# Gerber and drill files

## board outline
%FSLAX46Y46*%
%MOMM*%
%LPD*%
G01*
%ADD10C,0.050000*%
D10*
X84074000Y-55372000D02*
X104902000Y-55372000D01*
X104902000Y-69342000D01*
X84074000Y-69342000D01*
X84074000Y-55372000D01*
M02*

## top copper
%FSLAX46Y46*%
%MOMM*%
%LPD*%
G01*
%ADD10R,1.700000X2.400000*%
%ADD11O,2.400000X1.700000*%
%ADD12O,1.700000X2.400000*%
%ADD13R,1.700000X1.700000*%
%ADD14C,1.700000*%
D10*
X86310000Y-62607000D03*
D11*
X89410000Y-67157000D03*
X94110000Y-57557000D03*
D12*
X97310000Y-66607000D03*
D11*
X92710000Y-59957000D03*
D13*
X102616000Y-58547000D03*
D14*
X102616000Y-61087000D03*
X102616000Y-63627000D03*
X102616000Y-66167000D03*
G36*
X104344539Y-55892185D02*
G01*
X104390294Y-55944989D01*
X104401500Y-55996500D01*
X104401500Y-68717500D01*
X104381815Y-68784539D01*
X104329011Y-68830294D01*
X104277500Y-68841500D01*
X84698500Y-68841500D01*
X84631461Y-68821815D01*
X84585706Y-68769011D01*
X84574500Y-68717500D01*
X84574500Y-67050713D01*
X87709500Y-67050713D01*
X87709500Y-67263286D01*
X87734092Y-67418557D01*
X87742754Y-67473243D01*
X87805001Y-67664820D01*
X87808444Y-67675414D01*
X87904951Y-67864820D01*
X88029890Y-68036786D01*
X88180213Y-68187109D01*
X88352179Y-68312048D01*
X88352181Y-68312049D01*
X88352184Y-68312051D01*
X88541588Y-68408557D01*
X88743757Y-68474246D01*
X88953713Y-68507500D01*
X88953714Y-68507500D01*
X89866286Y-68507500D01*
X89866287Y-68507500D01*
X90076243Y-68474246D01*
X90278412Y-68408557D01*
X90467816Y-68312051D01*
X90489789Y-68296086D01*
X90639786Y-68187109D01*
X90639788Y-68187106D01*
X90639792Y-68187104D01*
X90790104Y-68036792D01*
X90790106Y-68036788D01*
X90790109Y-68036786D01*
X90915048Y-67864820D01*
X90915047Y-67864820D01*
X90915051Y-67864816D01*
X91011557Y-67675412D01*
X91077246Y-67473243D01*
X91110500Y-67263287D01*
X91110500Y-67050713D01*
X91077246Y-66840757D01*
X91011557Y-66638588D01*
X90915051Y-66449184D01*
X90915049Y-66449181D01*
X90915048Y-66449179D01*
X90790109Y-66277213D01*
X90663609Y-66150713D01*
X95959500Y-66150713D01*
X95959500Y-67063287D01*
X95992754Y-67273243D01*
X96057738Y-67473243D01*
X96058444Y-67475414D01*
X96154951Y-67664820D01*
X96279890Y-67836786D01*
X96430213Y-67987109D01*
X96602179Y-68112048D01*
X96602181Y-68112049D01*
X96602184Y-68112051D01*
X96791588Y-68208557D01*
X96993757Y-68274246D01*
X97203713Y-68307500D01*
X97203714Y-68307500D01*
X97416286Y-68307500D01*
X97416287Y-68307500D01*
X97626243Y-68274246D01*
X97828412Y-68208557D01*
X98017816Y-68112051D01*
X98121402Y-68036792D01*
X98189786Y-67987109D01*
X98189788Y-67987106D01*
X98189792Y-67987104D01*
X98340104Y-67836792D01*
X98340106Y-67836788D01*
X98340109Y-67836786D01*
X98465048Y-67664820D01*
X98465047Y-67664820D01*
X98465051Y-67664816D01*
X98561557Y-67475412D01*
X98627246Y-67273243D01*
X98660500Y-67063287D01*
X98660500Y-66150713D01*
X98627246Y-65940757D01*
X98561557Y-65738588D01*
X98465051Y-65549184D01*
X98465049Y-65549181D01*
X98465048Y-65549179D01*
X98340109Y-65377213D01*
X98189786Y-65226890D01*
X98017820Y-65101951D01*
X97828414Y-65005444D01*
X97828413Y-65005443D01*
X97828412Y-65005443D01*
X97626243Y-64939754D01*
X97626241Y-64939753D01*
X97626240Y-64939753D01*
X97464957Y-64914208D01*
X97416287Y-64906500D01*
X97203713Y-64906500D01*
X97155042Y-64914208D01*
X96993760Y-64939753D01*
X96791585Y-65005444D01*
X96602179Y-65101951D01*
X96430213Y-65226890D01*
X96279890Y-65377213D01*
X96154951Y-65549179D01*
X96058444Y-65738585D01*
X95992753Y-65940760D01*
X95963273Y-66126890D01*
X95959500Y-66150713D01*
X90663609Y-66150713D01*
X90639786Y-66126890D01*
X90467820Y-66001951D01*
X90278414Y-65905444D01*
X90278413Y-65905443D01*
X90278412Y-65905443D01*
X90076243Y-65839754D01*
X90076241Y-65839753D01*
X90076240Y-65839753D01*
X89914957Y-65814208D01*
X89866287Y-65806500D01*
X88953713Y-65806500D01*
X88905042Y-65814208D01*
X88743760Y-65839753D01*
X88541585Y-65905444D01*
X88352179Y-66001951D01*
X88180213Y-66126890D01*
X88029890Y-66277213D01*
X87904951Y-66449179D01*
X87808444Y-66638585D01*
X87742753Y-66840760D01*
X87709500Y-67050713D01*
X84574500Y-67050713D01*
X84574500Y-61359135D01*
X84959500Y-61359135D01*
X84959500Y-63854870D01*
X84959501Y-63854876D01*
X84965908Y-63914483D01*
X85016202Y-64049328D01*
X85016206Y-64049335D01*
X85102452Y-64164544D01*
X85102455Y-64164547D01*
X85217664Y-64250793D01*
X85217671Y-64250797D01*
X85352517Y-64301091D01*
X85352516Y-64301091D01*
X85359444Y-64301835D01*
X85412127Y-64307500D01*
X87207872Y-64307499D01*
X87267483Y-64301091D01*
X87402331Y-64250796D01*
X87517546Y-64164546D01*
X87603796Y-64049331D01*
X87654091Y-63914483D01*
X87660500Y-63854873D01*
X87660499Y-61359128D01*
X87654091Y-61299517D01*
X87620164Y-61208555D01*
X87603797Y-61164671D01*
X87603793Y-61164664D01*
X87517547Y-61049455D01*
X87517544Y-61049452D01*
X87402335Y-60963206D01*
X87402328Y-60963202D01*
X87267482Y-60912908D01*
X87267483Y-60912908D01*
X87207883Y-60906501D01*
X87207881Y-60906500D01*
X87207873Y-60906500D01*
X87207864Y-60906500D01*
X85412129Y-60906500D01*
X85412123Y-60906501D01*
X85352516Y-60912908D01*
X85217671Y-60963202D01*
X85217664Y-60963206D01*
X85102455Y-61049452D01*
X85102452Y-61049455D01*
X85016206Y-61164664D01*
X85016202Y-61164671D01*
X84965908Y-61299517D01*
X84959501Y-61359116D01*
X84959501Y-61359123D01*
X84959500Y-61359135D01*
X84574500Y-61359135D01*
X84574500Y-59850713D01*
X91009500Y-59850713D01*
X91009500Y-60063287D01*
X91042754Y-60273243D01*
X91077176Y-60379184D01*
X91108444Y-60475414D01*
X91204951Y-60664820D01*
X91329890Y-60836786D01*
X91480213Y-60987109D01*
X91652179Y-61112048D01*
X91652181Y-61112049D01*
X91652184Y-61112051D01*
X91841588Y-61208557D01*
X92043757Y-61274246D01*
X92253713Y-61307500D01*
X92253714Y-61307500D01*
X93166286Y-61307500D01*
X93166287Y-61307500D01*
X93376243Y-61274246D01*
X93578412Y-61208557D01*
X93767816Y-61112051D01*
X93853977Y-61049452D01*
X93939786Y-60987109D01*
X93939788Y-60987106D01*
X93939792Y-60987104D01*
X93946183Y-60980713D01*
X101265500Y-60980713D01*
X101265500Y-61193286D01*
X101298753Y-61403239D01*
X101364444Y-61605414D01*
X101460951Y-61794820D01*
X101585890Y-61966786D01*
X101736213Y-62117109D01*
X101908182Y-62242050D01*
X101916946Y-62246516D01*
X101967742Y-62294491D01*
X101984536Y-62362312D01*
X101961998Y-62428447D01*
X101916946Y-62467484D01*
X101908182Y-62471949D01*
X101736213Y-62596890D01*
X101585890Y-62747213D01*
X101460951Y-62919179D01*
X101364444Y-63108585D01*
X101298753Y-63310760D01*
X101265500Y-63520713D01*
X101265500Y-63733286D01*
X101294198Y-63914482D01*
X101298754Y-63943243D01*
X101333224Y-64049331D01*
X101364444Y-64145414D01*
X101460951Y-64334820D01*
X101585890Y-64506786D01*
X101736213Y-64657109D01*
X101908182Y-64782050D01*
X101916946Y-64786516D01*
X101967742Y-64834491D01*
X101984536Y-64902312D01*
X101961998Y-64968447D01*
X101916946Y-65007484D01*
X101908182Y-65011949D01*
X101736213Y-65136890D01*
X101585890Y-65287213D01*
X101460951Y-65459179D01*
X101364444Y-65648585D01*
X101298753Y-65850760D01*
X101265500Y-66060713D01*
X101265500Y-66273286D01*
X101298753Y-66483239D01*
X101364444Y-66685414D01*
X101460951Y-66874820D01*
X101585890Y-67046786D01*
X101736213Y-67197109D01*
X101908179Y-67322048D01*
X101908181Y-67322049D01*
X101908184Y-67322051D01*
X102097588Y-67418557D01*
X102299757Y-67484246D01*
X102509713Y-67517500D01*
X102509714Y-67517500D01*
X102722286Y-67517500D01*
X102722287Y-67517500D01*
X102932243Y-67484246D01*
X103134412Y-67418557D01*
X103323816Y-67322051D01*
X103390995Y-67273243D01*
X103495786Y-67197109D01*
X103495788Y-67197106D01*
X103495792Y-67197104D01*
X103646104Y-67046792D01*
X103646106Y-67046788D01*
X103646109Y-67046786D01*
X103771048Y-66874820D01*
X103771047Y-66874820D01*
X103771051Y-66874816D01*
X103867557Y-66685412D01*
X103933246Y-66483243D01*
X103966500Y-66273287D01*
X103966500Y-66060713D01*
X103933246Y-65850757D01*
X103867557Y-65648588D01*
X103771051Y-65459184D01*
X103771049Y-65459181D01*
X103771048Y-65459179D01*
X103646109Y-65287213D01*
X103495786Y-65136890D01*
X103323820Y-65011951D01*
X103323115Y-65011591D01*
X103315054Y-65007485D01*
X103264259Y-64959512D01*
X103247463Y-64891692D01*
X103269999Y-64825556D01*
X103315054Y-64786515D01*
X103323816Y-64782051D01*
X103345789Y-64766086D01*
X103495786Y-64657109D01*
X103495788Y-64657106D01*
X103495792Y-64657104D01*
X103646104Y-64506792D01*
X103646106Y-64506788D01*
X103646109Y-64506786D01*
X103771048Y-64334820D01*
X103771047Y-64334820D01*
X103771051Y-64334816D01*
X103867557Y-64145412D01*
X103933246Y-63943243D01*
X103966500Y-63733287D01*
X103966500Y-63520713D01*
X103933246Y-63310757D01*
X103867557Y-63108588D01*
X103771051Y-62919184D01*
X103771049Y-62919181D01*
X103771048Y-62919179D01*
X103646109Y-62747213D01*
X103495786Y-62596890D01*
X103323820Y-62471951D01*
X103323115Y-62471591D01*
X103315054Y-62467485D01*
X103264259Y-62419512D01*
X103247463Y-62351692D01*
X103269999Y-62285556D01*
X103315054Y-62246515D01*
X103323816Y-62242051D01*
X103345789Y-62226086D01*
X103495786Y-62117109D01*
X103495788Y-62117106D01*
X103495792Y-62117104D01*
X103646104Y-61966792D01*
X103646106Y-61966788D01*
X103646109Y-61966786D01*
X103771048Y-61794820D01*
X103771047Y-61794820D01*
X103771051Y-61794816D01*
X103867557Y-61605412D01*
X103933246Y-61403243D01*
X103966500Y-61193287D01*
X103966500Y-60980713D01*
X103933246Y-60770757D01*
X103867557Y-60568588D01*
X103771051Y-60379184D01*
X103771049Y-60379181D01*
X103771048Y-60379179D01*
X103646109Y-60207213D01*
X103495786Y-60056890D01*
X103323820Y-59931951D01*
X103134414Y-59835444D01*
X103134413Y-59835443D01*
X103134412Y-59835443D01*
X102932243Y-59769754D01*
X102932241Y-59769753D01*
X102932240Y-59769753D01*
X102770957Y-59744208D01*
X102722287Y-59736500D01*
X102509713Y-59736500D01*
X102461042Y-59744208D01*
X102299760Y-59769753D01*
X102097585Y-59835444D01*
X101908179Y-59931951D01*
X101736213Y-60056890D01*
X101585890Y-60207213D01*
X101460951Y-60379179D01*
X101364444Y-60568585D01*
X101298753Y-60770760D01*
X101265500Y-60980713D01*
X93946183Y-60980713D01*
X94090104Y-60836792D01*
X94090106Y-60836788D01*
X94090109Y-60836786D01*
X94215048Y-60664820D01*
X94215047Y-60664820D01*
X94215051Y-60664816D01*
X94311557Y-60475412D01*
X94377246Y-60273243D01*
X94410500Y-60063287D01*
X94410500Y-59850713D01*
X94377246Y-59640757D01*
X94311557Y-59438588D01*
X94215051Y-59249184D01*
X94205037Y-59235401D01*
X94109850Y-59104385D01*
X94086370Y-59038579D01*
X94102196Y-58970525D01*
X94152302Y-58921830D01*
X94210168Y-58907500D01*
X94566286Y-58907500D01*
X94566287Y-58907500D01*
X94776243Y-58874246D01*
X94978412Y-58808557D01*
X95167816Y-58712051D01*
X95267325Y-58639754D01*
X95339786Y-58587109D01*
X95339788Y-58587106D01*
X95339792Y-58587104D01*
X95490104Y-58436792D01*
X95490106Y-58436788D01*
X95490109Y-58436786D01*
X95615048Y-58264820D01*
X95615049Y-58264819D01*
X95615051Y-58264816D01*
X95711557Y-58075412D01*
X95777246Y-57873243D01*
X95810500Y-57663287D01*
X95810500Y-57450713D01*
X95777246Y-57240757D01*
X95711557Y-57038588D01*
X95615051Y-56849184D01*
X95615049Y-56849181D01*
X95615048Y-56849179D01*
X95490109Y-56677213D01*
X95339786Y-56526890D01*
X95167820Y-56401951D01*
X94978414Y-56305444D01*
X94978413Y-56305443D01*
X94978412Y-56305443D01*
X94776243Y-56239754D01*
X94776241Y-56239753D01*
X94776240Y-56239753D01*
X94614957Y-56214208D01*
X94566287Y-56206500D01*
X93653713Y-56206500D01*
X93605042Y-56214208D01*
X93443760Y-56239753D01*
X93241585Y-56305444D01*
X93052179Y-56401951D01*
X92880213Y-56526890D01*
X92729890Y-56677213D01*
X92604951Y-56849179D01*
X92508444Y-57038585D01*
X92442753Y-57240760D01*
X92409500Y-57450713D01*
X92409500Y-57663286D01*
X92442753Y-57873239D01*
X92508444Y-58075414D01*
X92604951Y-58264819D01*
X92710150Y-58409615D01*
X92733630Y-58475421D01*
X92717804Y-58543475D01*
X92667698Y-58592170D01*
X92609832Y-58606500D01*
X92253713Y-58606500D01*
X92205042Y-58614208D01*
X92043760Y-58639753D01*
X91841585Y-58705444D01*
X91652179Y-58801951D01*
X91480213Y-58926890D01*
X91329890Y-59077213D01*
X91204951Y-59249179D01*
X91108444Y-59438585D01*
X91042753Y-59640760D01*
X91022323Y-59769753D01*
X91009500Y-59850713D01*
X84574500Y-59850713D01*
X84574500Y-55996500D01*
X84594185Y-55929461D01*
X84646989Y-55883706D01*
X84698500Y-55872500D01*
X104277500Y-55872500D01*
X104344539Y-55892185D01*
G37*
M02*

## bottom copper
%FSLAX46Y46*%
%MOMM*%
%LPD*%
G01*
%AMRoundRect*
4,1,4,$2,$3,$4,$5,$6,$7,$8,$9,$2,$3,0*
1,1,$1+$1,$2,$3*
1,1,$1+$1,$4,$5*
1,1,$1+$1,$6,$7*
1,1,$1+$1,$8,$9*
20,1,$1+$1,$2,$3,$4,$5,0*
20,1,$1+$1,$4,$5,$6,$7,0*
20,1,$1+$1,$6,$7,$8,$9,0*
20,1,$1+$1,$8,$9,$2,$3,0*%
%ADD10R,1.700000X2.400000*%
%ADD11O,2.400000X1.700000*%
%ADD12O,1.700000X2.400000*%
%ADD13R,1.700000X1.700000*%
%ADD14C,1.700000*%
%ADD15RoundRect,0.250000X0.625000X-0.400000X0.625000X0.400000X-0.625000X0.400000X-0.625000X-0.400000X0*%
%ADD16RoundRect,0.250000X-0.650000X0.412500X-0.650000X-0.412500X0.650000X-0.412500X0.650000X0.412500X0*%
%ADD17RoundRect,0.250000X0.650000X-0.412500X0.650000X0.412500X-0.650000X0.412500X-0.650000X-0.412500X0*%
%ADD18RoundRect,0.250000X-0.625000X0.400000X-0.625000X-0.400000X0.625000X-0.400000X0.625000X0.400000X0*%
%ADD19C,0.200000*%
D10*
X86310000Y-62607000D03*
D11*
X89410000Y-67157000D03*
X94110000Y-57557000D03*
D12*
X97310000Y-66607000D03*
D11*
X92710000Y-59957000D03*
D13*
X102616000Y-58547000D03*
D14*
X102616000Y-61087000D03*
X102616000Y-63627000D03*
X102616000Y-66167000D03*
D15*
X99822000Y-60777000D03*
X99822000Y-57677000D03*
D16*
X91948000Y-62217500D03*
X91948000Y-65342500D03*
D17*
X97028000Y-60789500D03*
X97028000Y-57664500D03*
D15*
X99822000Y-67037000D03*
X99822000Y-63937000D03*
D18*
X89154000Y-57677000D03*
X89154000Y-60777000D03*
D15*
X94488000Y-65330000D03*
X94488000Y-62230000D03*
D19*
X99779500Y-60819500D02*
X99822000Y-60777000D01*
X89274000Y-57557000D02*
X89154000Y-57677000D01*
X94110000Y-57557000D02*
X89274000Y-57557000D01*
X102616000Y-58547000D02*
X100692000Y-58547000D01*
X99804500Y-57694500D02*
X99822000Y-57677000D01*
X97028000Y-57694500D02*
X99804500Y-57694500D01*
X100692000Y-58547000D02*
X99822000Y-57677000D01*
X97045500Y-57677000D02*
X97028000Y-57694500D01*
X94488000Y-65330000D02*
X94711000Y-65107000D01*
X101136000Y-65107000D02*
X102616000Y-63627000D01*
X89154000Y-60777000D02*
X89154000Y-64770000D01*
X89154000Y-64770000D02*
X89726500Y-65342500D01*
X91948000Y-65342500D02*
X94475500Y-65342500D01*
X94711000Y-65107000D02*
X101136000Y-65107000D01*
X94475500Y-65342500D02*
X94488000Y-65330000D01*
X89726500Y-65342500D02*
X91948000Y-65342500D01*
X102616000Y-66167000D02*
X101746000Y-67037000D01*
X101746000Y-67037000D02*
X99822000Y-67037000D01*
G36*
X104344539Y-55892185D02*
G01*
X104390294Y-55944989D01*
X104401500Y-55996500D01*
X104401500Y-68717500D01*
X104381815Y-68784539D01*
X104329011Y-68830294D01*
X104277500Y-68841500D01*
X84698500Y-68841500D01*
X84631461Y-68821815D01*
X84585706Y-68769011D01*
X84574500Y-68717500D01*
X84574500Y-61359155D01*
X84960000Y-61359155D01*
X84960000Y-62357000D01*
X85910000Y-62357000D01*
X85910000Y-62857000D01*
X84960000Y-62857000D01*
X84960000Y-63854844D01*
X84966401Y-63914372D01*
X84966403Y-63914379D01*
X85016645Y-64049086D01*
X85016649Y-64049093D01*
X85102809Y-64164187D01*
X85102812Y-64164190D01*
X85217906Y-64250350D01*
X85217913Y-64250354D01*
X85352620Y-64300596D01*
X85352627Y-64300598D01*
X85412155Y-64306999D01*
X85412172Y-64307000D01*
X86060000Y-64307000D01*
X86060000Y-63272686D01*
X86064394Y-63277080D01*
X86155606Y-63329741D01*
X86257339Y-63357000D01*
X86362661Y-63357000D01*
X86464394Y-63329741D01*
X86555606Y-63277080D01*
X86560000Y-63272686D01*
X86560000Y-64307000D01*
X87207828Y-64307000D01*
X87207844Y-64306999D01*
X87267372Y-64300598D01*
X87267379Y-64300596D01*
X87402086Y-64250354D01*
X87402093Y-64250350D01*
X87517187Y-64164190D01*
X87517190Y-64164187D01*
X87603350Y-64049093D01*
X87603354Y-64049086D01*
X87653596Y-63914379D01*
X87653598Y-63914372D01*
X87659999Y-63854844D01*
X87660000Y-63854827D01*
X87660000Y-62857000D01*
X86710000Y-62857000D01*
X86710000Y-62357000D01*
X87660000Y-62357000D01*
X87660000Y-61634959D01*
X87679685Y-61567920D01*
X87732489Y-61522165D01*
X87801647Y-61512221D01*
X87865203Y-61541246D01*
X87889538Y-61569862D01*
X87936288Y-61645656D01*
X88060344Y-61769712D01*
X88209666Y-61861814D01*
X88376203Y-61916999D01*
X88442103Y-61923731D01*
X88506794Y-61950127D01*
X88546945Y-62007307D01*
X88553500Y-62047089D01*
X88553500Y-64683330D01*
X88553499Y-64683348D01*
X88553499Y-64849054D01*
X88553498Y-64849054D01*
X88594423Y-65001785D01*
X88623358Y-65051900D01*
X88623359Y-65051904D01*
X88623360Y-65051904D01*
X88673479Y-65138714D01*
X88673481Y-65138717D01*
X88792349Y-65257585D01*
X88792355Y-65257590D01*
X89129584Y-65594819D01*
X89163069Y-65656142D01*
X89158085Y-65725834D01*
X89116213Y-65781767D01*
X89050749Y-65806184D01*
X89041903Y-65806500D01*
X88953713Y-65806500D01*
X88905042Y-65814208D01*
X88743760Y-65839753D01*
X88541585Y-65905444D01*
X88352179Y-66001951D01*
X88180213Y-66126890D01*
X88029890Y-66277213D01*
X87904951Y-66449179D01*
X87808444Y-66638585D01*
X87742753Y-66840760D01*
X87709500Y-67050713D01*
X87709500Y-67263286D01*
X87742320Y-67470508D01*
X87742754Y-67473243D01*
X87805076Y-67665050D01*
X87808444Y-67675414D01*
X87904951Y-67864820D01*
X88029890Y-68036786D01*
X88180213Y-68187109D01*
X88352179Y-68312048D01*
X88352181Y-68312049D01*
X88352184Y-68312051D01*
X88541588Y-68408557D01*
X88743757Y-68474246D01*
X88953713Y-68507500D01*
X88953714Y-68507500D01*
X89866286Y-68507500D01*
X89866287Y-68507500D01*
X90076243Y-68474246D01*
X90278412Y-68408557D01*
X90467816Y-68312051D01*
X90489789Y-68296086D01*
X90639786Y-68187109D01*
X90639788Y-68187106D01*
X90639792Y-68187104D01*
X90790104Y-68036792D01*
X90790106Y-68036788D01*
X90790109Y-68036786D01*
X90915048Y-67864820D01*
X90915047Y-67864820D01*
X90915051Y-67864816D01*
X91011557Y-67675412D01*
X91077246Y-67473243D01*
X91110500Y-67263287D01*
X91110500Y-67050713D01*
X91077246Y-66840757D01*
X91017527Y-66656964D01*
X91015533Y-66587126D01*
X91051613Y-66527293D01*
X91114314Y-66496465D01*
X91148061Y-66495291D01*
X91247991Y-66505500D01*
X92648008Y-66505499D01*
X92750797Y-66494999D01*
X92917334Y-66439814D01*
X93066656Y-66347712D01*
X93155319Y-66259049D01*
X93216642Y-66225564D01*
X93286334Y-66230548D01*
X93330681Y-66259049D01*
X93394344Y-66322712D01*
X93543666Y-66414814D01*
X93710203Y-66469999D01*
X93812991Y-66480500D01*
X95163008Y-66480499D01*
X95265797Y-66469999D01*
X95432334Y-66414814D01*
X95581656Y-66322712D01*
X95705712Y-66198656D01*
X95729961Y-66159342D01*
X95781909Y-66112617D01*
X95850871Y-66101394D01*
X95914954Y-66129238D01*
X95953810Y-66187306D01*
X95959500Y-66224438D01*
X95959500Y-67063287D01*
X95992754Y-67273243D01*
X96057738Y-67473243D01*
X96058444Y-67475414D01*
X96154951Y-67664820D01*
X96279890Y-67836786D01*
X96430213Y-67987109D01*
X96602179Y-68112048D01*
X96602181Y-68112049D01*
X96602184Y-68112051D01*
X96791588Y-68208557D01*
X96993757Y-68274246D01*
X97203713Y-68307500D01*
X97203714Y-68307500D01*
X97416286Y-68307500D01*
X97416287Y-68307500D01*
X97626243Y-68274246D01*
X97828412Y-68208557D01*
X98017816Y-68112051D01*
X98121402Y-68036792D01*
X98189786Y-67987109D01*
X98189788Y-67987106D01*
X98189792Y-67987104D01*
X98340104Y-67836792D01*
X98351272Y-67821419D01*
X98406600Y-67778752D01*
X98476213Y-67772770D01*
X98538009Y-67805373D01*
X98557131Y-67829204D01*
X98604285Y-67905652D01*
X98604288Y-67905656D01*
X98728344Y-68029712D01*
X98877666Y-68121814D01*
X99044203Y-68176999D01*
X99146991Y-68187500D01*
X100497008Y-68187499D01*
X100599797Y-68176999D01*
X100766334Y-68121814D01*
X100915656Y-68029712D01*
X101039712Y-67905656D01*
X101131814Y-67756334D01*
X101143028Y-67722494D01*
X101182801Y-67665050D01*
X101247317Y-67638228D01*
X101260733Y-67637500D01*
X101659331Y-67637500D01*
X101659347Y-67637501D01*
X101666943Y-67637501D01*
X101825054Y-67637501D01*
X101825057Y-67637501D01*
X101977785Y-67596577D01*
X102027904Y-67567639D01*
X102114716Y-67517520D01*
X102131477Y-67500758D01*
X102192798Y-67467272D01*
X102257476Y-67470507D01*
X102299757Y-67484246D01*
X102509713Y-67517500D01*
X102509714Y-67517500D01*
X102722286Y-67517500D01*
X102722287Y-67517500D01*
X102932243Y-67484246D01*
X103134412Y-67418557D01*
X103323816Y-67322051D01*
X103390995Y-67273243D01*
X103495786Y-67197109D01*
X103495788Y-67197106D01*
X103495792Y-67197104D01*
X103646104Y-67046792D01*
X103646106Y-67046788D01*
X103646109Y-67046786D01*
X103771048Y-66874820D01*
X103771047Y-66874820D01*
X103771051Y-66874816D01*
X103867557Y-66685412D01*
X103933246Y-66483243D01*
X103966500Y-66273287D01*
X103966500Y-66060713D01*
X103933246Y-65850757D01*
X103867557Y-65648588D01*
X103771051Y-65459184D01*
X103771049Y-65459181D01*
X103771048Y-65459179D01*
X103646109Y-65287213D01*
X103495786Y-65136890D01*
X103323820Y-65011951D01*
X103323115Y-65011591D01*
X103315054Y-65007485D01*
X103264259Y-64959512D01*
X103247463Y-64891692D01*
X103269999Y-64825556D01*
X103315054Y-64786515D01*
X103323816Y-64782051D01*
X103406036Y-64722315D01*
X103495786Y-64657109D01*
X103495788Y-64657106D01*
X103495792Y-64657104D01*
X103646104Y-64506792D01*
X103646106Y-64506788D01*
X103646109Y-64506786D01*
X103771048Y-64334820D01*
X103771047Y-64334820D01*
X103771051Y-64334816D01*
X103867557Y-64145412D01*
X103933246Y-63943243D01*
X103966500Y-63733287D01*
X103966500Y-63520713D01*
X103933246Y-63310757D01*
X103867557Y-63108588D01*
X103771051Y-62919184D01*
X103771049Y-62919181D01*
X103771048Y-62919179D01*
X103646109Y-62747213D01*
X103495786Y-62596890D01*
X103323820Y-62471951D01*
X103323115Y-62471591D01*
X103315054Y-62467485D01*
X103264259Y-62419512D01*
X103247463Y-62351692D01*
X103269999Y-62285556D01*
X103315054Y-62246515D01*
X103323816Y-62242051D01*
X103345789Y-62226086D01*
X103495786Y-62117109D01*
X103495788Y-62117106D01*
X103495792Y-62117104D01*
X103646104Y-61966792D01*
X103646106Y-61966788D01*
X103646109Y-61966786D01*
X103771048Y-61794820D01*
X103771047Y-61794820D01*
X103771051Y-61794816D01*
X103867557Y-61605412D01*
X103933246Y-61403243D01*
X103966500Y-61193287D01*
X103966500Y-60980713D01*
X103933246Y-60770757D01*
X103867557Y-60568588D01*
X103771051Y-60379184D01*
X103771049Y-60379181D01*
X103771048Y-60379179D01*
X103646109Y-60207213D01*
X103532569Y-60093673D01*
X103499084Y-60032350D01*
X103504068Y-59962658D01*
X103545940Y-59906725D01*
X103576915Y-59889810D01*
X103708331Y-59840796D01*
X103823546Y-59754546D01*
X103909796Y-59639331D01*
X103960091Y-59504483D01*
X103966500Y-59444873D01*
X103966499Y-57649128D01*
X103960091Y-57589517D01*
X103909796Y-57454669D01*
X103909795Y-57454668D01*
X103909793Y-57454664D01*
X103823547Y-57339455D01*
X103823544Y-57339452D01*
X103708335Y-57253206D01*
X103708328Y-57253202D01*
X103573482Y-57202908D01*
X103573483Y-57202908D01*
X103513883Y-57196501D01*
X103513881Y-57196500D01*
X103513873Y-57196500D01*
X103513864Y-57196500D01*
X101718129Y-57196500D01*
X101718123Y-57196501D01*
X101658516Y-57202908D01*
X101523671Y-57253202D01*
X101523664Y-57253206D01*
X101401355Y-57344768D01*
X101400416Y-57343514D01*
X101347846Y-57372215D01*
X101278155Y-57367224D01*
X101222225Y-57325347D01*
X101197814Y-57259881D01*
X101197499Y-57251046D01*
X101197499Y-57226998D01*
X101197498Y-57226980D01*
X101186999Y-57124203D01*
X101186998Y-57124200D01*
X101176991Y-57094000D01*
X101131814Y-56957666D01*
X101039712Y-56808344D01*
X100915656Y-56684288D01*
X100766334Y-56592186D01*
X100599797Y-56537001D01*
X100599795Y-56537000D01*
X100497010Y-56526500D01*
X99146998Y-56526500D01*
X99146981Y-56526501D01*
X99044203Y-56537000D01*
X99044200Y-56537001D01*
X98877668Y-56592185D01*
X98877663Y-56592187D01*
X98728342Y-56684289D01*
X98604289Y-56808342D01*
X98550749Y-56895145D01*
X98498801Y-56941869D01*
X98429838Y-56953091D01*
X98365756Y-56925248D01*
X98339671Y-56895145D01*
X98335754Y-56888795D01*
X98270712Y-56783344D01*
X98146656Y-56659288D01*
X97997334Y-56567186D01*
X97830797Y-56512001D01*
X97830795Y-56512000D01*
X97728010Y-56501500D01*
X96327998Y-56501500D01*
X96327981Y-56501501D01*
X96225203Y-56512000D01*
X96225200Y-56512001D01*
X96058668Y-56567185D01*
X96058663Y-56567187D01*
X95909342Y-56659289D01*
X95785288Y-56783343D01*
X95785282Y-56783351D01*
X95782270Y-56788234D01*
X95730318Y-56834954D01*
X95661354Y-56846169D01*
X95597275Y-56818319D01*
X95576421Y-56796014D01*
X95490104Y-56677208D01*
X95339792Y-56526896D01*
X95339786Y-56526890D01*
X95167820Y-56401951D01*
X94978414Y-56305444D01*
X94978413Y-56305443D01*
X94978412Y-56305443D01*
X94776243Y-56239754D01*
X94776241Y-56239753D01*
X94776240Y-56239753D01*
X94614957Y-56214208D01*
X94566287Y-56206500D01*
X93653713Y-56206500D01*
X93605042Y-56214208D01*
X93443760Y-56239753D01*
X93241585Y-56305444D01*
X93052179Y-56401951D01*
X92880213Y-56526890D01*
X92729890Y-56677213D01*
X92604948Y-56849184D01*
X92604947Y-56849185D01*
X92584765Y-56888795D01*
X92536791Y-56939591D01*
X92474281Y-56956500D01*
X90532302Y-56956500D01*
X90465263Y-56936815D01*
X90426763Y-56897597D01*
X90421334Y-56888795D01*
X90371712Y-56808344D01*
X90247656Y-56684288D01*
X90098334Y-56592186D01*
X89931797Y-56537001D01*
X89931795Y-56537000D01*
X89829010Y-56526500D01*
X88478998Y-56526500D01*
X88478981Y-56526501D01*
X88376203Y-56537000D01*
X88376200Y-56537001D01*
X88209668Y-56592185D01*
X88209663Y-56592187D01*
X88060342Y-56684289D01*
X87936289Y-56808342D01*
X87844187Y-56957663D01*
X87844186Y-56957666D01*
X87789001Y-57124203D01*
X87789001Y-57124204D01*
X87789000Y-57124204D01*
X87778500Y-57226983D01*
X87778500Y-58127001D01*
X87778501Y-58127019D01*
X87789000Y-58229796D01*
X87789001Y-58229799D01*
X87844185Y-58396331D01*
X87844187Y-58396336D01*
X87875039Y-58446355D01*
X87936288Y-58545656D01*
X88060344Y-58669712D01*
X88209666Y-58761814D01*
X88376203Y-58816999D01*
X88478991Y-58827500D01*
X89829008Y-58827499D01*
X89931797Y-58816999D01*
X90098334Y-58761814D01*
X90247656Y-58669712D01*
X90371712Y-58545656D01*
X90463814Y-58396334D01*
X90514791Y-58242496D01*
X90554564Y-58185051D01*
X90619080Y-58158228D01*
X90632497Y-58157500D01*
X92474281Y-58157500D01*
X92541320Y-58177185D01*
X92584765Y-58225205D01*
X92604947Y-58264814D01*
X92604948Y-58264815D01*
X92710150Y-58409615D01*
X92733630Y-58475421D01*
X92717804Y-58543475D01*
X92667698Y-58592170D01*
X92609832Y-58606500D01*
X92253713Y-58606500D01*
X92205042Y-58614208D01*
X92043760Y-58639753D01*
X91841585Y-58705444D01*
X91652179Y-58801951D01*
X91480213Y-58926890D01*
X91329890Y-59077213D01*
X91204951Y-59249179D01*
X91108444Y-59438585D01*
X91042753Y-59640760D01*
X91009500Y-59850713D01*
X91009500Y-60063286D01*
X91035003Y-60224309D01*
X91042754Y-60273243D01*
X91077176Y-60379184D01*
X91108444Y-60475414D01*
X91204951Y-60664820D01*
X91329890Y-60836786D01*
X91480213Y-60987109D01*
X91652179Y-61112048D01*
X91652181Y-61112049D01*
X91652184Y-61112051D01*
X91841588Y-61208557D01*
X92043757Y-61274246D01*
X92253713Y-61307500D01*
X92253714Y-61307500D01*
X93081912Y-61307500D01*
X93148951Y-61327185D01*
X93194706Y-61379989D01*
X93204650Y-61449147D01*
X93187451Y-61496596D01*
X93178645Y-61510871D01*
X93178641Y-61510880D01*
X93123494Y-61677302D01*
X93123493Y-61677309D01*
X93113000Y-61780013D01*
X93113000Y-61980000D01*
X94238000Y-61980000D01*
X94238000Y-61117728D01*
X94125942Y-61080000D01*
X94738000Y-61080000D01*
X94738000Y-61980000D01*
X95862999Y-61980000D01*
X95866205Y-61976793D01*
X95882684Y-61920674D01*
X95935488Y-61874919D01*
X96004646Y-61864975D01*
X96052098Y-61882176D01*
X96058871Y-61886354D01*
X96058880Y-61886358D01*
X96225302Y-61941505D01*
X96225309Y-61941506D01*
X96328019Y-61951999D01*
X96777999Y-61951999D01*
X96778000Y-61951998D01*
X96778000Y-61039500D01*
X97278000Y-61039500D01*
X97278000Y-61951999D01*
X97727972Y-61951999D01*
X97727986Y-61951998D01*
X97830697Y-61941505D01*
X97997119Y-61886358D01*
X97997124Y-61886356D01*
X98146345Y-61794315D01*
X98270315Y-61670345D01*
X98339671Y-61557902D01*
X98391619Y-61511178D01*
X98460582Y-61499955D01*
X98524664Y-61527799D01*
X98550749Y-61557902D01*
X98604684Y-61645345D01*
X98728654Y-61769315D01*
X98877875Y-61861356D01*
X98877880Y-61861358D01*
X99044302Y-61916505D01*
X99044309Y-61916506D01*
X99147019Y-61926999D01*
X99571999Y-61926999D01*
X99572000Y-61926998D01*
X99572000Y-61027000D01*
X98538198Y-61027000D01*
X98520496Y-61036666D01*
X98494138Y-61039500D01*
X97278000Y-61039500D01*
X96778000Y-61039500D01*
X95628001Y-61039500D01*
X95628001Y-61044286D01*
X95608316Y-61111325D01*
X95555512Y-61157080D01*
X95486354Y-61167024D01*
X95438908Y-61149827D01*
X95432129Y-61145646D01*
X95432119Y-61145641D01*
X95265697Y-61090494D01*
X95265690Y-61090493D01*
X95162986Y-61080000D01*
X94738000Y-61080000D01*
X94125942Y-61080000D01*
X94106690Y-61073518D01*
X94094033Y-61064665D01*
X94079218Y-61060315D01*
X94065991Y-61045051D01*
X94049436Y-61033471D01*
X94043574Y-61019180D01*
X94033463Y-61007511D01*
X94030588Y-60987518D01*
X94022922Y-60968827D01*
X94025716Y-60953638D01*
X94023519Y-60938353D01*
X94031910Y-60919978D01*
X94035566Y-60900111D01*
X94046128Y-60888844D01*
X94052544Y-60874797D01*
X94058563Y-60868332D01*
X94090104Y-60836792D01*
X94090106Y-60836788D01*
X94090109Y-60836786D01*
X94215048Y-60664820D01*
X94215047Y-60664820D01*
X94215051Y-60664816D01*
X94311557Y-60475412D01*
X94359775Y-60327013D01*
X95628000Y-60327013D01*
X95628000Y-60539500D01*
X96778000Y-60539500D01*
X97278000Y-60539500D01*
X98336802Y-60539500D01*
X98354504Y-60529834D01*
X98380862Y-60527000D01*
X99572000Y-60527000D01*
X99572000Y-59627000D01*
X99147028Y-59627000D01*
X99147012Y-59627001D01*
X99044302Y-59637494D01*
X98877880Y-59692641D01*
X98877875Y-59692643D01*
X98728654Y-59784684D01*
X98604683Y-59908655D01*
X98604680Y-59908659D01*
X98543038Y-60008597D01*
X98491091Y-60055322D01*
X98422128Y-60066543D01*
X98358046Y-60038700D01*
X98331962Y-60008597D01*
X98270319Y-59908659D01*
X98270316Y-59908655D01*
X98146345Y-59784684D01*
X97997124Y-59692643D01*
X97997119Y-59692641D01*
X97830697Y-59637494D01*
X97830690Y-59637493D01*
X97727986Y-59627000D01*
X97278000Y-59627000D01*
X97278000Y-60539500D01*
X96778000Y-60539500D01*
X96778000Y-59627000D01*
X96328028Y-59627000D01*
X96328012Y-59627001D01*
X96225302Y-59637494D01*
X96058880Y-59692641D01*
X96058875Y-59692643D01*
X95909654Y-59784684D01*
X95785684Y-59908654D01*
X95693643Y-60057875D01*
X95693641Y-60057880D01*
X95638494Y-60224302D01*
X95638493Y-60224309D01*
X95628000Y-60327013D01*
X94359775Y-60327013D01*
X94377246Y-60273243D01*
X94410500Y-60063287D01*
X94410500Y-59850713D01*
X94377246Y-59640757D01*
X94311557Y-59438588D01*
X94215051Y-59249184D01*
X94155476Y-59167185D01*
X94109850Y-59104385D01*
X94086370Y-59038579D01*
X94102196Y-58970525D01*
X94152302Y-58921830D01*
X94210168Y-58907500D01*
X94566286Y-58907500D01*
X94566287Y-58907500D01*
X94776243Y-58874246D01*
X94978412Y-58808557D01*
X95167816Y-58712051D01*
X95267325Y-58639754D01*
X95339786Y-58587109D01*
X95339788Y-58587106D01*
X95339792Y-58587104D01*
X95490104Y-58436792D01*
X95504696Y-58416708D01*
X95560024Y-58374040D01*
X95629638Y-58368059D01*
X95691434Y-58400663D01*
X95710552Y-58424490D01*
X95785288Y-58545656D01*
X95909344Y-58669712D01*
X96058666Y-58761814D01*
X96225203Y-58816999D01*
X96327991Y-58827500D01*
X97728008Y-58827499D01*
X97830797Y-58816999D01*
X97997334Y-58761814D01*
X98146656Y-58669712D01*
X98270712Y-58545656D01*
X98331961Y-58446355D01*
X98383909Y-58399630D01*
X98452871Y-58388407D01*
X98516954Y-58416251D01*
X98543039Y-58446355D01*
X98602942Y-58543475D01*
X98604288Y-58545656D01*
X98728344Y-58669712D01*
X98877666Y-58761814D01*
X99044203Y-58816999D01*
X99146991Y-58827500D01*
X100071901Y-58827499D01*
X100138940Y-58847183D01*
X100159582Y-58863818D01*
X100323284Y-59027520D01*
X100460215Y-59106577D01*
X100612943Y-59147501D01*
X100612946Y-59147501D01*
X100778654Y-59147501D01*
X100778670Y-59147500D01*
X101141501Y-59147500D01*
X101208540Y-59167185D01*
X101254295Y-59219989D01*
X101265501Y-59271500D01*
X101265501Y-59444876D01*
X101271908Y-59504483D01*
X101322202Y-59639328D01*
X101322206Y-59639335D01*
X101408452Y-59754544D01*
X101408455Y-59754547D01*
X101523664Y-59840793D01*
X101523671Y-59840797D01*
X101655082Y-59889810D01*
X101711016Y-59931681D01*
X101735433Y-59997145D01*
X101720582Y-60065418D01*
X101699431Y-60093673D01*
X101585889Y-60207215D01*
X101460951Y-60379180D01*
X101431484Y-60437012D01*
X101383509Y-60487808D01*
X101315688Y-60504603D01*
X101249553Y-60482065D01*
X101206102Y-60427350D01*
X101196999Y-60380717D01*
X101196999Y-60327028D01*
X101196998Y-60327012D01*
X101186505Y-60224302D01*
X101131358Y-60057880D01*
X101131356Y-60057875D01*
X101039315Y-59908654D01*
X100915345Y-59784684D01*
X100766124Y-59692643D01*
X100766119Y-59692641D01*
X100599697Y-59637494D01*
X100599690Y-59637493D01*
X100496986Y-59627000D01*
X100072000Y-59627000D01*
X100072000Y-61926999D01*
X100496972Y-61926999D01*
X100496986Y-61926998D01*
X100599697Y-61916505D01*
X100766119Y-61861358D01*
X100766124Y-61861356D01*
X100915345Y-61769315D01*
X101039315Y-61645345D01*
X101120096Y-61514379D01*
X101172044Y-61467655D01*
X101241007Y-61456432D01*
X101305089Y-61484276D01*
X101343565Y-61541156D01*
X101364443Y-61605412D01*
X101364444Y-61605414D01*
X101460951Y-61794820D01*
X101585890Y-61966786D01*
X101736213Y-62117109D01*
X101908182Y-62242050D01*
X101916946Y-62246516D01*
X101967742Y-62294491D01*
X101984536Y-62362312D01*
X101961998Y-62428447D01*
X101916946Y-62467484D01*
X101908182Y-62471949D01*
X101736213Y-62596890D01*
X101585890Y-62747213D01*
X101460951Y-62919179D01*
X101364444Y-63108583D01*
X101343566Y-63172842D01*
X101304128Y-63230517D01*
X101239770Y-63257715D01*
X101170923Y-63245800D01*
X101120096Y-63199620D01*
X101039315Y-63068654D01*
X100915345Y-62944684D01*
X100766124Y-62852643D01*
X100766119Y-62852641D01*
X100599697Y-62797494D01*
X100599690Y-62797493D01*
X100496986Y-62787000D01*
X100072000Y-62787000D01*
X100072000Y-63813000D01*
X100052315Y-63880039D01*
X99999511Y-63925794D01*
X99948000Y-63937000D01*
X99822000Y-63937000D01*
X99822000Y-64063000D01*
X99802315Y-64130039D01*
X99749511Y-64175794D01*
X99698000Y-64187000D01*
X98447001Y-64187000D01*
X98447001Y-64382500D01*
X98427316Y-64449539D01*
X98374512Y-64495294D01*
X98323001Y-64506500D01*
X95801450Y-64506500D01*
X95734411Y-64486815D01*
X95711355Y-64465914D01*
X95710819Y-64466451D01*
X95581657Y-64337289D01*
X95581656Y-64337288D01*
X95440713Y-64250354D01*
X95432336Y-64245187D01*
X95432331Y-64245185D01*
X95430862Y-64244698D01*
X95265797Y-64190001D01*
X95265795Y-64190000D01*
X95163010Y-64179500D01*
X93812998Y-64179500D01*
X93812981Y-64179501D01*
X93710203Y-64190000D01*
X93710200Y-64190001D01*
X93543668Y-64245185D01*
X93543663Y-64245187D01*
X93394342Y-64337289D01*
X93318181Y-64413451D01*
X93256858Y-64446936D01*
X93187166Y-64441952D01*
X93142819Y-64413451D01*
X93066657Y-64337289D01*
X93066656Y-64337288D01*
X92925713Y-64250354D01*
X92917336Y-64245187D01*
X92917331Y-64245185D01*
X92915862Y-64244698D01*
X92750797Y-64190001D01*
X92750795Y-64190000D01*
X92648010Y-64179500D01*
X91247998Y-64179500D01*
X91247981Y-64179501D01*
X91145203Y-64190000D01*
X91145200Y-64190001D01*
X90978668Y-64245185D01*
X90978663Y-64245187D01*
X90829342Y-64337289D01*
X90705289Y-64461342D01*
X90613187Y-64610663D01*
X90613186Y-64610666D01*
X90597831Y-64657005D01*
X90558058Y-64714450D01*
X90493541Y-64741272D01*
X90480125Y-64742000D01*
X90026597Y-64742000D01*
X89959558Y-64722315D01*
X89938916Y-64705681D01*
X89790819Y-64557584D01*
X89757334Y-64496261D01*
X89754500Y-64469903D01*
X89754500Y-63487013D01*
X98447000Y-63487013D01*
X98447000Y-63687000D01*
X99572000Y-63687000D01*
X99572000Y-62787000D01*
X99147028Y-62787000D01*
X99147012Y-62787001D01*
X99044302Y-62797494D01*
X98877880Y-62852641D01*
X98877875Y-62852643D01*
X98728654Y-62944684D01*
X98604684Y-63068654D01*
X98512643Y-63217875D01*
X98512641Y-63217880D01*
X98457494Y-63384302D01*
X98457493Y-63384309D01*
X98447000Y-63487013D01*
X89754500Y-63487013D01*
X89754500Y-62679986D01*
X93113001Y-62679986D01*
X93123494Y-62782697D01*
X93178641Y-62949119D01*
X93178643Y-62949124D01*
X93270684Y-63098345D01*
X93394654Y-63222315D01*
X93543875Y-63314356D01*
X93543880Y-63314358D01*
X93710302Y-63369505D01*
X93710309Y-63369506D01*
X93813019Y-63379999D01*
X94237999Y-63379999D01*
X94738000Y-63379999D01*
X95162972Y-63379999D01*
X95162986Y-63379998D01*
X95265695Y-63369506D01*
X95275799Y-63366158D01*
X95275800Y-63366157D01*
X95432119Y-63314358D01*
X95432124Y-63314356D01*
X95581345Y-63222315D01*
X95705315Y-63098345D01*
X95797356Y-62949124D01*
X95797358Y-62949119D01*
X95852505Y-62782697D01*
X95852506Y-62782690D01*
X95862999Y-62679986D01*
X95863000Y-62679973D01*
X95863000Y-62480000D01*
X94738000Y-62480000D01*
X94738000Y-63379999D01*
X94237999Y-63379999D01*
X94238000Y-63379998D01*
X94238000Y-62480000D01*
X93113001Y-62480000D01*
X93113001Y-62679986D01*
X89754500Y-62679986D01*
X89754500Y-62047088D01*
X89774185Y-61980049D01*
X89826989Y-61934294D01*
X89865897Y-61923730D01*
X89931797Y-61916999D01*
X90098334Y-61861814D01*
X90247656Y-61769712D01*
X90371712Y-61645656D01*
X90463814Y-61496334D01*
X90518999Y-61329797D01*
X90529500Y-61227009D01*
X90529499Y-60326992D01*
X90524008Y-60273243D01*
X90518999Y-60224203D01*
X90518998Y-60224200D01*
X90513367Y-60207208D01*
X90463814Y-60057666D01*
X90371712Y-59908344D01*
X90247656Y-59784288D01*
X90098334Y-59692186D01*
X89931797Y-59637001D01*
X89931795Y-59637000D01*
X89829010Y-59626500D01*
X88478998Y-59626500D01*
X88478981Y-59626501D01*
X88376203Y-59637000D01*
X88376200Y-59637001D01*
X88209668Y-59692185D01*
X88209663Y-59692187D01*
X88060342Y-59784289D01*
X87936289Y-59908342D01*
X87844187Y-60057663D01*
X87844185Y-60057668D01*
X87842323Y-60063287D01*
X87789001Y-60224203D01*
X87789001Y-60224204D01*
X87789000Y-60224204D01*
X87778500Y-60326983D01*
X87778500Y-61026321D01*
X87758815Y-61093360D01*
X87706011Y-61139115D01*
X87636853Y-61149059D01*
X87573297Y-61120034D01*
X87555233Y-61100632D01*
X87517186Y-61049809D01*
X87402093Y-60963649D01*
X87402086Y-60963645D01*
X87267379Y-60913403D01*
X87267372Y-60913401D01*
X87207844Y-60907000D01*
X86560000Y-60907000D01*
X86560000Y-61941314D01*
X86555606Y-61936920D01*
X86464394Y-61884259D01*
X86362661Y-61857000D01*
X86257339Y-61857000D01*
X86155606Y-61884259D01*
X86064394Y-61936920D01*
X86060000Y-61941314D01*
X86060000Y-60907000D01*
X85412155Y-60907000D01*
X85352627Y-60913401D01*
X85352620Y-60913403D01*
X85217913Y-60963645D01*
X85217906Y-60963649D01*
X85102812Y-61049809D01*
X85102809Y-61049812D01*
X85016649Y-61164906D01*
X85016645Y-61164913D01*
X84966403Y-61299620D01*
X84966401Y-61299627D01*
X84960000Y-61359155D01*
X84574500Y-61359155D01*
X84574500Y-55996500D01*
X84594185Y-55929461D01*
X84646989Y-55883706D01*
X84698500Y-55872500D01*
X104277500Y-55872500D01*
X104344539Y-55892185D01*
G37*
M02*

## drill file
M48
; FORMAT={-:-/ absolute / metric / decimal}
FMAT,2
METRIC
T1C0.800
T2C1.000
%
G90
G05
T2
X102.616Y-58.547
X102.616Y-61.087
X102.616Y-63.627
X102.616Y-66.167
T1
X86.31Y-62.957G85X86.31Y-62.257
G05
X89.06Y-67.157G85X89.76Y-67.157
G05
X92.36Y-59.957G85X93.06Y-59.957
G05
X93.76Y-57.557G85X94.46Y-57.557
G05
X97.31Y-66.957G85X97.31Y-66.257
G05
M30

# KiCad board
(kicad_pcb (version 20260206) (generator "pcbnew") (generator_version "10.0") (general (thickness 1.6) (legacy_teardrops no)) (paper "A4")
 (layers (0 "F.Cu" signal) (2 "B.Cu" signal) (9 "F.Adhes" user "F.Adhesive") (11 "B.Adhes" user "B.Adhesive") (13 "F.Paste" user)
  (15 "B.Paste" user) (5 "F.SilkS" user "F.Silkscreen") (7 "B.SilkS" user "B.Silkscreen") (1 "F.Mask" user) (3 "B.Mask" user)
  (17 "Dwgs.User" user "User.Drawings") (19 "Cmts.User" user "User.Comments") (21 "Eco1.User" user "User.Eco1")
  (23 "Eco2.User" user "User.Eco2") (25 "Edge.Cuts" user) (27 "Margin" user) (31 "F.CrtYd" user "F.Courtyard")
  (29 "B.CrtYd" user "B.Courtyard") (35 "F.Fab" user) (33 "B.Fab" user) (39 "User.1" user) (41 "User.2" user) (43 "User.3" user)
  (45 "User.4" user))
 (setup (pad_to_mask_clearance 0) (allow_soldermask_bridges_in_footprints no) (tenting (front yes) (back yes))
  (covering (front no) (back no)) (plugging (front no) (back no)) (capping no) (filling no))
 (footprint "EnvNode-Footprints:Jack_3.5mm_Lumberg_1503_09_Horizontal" (layer "F.Cu") (at 86.31 62.607 90)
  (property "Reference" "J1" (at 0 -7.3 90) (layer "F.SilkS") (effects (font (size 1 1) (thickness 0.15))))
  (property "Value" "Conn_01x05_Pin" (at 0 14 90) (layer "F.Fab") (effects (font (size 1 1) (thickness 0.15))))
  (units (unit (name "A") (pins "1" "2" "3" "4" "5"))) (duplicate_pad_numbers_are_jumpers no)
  (pad "1" thru_hole rect (at 0 0 90) (size 2.4 1.7) (drill oval 1.5 0.8) (layers "*.Cu" "*.Mask") (remove_unused_layers no) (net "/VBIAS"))
  (pad "2" thru_hole oval (at -4.55 3.1 90) (size 1.7 2.4) (drill oval 0.8 1.5) (layers "*.Cu" "*.Mask") (remove_unused_layers no)
   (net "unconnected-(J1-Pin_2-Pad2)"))
  (pad "3" thru_hole oval (at 5.05 7.8 90) (size 1.7 2.4) (drill oval 0.8 1.5) (layers "*.Cu" "*.Mask") (remove_unused_layers no)
   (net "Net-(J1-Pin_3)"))
  (pad "4" thru_hole oval (at -4 11 90) (size 2.4 1.7) (drill oval 1.5 0.8) (layers "*.Cu" "*.Mask") (remove_unused_layers no)
   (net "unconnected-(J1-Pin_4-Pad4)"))
  (pad "5" thru_hole oval (at 2.65 6.4 90) (size 1.7 2.4) (drill oval 0.8 1.5) (layers "*.Cu" "*.Mask") (remove_unused_layers no)
   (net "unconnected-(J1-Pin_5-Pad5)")))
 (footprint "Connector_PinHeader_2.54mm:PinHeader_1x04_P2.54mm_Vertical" (layer "F.Cu") (at 102.616 58.547)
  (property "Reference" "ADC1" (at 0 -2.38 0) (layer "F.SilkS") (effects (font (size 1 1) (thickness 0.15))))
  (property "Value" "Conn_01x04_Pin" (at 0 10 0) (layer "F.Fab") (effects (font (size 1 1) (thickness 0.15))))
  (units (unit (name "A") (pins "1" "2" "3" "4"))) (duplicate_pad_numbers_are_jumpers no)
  (pad "1" thru_hole rect (at 0 0) (size 1.7 1.7) (drill 1) (layers "*.Cu" "*.Mask") (remove_unused_layers no) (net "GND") (zone_connect 2))
  (pad "2" thru_hole circle (at 0 2.54) (size 1.7 1.7) (drill 1) (layers "*.Cu" "*.Mask") (remove_unused_layers no)
   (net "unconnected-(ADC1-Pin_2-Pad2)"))
  (pad "3" thru_hole circle (at 0 5.08) (size 1.7 1.7) (drill 1) (layers "*.Cu" "*.Mask") (remove_unused_layers no) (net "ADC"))
  (pad "4" thru_hole circle (at 0 7.62) (size 1.7 1.7) (drill 1) (layers "*.Cu" "*.Mask") (remove_unused_layers no) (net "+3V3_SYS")))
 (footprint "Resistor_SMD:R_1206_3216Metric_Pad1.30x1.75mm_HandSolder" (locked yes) (layer "B.Cu") (at 99.822 59.227 90)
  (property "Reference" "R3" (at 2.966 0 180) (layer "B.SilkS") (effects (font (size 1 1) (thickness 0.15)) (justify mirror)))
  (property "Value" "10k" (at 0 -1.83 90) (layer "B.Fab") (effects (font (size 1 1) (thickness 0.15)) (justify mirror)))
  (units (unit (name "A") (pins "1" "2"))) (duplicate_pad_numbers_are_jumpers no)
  (pad "1" smd roundrect (at -1.55 0 90) (size 1.3 1.75) (layers "B.Cu" "B.Mask" "B.Paste") (roundrect_rratio 0.192308) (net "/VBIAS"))
  (pad "2" smd roundrect (at 1.55 0 90) (size 1.3 1.75) (layers "B.Cu" "B.Mask" "B.Paste") (roundrect_rratio 0.192308) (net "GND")))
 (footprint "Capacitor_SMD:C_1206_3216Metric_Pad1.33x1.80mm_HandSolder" (layer "B.Cu") (at 91.948 63.78 -90)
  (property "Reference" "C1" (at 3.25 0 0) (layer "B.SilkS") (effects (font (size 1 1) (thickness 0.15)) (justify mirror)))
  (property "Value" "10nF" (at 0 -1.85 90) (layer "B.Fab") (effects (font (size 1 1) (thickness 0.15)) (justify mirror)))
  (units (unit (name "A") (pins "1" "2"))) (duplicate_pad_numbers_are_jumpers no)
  (pad "1" smd roundrect (at -1.5625 0 270) (size 1.325 1.8) (layers "B.Cu" "B.Mask" "B.Paste") (roundrect_rratio 0.188679) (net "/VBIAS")
   (zone_connect 2))
  (pad "2" smd roundrect (at 1.5625 0 270) (size 1.325 1.8) (layers "B.Cu" "B.Mask" "B.Paste") (roundrect_rratio 0.188679) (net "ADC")))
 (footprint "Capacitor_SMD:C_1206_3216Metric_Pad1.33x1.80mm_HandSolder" (layer "B.Cu") (at 97.028 59.227 90)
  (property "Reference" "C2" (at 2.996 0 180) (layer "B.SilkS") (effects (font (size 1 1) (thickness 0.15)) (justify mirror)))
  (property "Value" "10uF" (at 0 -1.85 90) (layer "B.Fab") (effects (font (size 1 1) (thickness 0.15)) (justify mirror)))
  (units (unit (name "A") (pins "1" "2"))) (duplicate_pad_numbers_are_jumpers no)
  (pad "1" smd roundrect (at -1.5625 0 90) (size 1.325 1.8) (layers "B.Cu" "B.Mask" "B.Paste") (roundrect_rratio 0.188679) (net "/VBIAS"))
  (pad "2" smd roundrect (at 1.5625 0 90) (size 1.325 1.8) (layers "B.Cu" "B.Mask" "B.Paste") (roundrect_rratio 0.188679) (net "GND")))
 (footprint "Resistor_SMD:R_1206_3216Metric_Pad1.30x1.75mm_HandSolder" (layer "B.Cu") (at 99.822 65.487 90)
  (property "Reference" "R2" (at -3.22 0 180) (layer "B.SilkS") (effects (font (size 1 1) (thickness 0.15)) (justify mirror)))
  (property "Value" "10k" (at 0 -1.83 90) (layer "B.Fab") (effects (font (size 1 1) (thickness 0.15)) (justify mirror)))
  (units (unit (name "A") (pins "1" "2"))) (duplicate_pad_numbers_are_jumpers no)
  (pad "1" smd roundrect (at -1.55 0 90) (size 1.3 1.75) (layers "B.Cu" "B.Mask" "B.Paste") (roundrect_rratio 0.192308) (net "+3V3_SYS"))
  (pad "2" smd roundrect (at 1.55 0 90) (size 1.3 1.75) (layers "B.Cu" "B.Mask" "B.Paste") (roundrect_rratio 0.192308) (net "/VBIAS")))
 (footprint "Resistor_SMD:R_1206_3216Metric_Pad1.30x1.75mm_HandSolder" (layer "B.Cu") (at 89.154 59.227 -90)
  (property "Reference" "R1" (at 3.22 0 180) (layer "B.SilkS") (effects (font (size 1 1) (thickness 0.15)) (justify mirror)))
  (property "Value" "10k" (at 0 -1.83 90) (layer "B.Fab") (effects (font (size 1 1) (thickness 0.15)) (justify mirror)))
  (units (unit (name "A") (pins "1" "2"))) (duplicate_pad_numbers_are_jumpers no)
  (pad "1" smd roundrect (at -1.55 0 270) (size 1.3 1.75) (layers "B.Cu" "B.Mask" "B.Paste") (roundrect_rratio 0.192308)
   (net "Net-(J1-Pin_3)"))
  (pad "2" smd roundrect (at 1.55 0 270) (size 1.3 1.75) (layers "B.Cu" "B.Mask" "B.Paste") (roundrect_rratio 0.192308) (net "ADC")))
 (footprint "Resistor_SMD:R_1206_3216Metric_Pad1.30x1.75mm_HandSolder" (layer "B.Cu") (at 94.488 63.78 90)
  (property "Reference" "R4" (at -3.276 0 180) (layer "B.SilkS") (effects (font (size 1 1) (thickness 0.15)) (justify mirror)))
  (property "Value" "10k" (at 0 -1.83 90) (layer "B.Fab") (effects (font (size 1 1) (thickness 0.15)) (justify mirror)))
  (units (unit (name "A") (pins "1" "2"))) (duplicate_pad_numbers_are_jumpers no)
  (pad "1" smd roundrect (at -1.55 0 90) (size 1.3 1.75) (layers "B.Cu" "B.Mask" "B.Paste") (roundrect_rratio 0.192308) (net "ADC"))
  (pad "2" smd roundrect (at 1.55 0 90) (size 1.3 1.75) (layers "B.Cu" "B.Mask" "B.Paste") (roundrect_rratio 0.192308) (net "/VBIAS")))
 (gr_rect (start 84.074 55.372) (end 104.902 69.342) (stroke (width 0.05) (type default)) (fill no) (layer "Edge.Cuts"))
 (segment (start 99.7795 60.8195) (end 99.822 60.777) (width 0.2) (layer "B.Cu") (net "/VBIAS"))
 (segment (start 89.274 57.557) (end 89.154 57.677) (width 0.2) (layer "B.Cu") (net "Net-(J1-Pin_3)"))
 (segment (start 94.11 57.557) (end 89.274 57.557) (width 0.2) (layer "B.Cu") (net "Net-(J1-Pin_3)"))
 (segment (start 102.616 58.547) (end 100.692 58.547) (width 0.2) (layer "B.Cu") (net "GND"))
 (segment (start 99.8045 57.6945) (end 99.822 57.677) (width 0.2) (layer "B.Cu") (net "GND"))
 (segment (start 97.028 57.6945) (end 99.8045 57.6945) (width 0.2) (layer "B.Cu") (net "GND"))
 (segment (start 100.692 58.547) (end 99.822 57.677) (width 0.2) (layer "B.Cu") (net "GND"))
 (segment (start 97.0455 57.677) (end 97.028 57.6945) (width 0.2) (layer "B.Cu") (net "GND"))
 (segment (start 94.488 65.33) (end 94.711 65.107) (width 0.2) (layer "B.Cu") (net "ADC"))
 (segment (start 101.136 65.107) (end 102.616 63.627) (width 0.2) (layer "B.Cu") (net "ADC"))
 (segment (start 89.154 60.777) (end 89.154 64.77) (width 0.2) (layer "B.Cu") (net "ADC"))
 (segment (start 89.154 64.77) (end 89.7265 65.3425) (width 0.2) (layer "B.Cu") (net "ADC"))
 (segment (start 91.948 65.3425) (end 94.4755 65.3425) (width 0.2) (layer "B.Cu") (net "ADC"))
 (segment (start 94.711 65.107) (end 101.136 65.107) (width 0.2) (layer "B.Cu") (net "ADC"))
 (segment (start 94.4755 65.3425) (end 94.488 65.33) (width 0.2) (layer "B.Cu") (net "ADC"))
 (segment (start 89.7265 65.3425) (end 91.948 65.3425) (width 0.2) (layer "B.Cu") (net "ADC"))
 (segment (start 102.616 66.167) (end 101.746 67.037) (width 0.2) (layer "B.Cu") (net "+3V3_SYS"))
 (segment (start 101.746 67.037) (end 99.822 67.037) (width 0.2) (layer "B.Cu") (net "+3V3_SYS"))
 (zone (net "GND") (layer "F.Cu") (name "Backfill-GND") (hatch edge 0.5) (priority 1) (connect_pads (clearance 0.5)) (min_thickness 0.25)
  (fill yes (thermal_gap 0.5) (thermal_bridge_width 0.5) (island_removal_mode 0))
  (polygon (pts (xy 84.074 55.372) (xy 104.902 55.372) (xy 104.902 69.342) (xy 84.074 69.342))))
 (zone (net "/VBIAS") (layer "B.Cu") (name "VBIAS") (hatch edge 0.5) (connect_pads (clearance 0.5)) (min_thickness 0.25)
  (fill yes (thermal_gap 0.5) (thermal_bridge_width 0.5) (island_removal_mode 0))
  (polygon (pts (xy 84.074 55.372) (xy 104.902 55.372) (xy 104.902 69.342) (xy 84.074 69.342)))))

